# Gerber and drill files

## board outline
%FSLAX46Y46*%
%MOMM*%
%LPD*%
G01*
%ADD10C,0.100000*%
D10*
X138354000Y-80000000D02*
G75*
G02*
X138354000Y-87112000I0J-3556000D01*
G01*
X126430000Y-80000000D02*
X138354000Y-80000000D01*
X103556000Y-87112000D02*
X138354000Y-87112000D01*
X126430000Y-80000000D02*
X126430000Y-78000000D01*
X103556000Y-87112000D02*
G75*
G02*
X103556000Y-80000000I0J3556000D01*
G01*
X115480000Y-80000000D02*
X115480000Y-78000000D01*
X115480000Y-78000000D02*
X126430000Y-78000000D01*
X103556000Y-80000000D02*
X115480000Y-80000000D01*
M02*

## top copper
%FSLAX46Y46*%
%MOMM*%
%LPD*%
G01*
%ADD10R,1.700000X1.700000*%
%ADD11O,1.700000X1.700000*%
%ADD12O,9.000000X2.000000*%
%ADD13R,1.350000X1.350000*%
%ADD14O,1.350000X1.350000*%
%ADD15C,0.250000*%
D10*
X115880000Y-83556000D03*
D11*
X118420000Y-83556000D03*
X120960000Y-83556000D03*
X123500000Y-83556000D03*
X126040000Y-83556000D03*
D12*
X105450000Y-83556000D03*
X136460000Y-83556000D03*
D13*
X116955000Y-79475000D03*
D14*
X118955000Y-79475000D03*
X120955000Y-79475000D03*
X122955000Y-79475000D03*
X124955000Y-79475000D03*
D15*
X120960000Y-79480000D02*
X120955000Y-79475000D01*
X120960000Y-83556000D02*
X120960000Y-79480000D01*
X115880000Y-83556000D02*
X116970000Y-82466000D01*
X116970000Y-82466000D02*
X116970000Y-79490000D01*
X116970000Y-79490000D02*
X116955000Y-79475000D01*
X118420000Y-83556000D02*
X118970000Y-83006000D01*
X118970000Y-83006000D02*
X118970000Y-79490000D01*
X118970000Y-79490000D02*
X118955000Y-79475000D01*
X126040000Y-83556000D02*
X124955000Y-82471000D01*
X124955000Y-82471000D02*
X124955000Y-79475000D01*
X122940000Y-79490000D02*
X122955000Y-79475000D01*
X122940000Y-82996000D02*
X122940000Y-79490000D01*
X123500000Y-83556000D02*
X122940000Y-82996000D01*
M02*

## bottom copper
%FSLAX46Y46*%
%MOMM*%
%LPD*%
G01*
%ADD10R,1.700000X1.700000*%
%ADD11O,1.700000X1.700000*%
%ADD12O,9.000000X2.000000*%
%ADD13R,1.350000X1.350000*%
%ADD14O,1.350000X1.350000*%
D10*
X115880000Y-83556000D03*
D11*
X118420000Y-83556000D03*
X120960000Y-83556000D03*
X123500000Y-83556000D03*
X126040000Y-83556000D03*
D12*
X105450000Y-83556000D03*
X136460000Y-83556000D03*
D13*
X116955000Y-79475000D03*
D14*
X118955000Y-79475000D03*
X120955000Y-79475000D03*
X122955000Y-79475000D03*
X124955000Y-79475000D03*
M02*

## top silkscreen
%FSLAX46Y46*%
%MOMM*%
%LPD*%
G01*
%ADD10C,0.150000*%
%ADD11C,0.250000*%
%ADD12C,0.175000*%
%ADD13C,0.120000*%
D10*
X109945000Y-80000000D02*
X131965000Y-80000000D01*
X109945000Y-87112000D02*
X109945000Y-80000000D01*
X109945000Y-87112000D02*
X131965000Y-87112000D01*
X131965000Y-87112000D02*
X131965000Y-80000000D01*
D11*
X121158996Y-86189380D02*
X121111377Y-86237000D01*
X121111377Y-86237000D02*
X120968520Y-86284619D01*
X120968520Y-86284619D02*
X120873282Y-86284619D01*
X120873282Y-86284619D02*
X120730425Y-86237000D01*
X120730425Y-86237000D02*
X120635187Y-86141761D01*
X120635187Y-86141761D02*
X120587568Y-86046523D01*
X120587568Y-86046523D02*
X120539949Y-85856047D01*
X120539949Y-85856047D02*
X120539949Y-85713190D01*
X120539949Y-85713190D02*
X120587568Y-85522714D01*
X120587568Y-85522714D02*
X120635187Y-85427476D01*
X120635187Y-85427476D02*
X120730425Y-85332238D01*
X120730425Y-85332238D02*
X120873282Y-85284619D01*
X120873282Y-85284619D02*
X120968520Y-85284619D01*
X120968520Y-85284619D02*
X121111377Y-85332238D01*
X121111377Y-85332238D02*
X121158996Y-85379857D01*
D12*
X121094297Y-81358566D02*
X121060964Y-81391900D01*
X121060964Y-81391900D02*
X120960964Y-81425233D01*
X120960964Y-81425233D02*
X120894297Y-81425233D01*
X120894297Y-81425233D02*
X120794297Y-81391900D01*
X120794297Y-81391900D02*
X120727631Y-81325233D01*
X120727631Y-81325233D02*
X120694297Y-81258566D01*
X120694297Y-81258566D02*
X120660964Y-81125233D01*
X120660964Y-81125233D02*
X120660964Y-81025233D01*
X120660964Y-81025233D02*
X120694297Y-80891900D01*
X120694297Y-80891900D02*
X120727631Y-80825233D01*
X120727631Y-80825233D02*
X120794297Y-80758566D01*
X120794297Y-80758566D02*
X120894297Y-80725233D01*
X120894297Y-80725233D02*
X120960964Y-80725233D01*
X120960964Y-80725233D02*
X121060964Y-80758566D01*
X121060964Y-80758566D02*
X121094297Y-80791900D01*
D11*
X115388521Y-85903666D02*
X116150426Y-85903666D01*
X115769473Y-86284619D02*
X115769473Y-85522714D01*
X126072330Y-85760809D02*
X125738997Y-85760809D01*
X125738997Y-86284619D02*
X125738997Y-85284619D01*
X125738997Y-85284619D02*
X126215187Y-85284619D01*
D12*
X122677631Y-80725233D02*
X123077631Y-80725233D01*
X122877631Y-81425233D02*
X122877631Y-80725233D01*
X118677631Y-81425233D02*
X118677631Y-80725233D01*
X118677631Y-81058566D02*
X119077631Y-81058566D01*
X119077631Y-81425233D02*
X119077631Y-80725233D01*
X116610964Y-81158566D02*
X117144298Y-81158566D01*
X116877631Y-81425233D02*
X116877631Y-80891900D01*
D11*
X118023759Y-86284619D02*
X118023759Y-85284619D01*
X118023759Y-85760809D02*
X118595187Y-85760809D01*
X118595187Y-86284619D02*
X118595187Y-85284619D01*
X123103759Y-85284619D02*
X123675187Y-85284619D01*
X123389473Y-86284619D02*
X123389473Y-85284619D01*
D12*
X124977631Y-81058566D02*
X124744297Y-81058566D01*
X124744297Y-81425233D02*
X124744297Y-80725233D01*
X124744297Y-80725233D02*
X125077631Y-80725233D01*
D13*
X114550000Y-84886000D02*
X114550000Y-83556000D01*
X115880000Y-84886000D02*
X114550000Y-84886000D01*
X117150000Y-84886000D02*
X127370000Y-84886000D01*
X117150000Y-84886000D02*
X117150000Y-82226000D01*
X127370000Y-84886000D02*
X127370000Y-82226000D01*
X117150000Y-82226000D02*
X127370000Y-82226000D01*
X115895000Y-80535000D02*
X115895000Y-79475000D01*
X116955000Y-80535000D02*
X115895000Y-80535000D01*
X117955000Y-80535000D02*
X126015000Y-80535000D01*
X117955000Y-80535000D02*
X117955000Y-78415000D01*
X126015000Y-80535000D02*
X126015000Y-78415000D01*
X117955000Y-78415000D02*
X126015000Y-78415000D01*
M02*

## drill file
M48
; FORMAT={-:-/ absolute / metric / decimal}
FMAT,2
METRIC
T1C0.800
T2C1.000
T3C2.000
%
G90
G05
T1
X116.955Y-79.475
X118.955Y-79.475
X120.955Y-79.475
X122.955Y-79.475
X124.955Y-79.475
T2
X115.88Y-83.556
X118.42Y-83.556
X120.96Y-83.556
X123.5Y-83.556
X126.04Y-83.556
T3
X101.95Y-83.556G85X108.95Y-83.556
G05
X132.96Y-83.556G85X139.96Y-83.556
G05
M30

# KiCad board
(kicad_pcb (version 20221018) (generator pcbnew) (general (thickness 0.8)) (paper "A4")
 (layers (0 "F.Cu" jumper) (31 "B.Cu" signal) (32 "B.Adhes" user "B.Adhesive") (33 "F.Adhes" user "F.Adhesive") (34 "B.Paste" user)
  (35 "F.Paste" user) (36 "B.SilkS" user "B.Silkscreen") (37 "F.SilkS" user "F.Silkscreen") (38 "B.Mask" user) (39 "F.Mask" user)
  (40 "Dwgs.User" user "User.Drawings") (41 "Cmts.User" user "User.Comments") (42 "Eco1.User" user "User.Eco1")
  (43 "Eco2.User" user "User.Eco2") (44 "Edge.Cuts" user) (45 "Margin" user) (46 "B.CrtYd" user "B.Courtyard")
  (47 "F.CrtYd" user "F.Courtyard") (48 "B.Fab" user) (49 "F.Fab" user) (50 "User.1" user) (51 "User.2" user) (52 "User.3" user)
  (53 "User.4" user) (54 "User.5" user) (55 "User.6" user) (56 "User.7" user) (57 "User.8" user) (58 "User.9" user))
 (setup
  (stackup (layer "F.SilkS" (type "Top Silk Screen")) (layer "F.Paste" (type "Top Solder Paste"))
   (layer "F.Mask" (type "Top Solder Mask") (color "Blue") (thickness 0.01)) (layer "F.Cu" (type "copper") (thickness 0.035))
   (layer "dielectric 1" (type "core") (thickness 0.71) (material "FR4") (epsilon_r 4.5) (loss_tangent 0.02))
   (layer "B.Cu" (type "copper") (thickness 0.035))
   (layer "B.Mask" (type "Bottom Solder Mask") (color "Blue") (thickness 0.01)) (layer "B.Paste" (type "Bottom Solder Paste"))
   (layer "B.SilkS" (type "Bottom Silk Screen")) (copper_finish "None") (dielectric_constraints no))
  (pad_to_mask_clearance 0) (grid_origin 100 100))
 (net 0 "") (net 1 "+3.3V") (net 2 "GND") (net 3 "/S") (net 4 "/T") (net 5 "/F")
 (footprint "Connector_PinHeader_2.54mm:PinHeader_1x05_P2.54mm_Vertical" (layer "F.Cu") (at 115.88 83.556 90)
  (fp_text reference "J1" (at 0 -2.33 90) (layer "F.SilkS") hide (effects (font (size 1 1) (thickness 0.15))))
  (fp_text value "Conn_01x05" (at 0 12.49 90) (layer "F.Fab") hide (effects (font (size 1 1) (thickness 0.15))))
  (fp_line (start -1.33 -1.33) (end 0 -1.33) (stroke (width 0.12) (type solid)) (layer "F.SilkS"))
  (fp_line (start -1.33 0) (end -1.33 -1.33) (stroke (width 0.12) (type solid)) (layer "F.SilkS"))
  (fp_line (start -1.33 1.27) (end -1.33 11.49) (stroke (width 0.12) (type solid)) (layer "F.SilkS"))
  (fp_line (start -1.33 1.27) (end 1.33 1.27) (stroke (width 0.12) (type solid)) (layer "F.SilkS"))
  (fp_line (start -1.33 11.49) (end 1.33 11.49) (stroke (width 0.12) (type solid)) (layer "F.SilkS"))
  (fp_line (start 1.33 1.27) (end 1.33 11.49) (stroke (width 0.12) (type solid)) (layer "F.SilkS"))
  (pad "1" thru_hole rect (at 0 0 90) (size 1.7 1.7) (drill 1) (layers "*.Cu" "*.Mask") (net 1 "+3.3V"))
  (pad "2" thru_hole oval (at 0 2.54 90) (size 1.7 1.7) (drill 1) (layers "*.Cu" "*.Mask") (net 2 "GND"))
  (pad "3" thru_hole oval (at 0 5.08 90) (size 1.7 1.7) (drill 1) (layers "*.Cu" "*.Mask") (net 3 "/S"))
  (pad "4" thru_hole oval (at 0 7.62 90) (size 1.7 1.7) (drill 1) (layers "*.Cu" "*.Mask") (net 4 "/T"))
  (pad "5" thru_hole oval (at 0 10.16 90) (size 1.7 1.7) (drill 1) (layers "*.Cu" "*.Mask") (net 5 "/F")))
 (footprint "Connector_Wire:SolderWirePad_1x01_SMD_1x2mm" (layer "F.Cu") (at 105.45 83.556)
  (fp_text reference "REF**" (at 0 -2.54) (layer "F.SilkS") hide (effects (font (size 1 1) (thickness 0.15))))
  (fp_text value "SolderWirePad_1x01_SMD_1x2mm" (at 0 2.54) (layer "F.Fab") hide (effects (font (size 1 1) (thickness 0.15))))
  (pad "1" thru_hole oval (at 0 0) (size 9 2) (drill oval 9 2) (layers "*.Cu" "*.Mask")))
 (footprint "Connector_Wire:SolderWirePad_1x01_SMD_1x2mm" (layer "F.Cu") (at 136.46 83.556)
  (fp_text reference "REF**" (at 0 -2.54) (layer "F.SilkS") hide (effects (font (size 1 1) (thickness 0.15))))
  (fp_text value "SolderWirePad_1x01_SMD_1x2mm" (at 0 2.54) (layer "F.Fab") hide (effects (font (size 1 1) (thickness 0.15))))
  (pad "1" thru_hole oval (at 0 0) (size 9 2) (drill oval 9 2) (layers "*.Cu" "*.Mask")))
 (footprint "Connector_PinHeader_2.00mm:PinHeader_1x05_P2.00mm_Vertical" (layer "F.Cu") (at 116.955 79.475 90)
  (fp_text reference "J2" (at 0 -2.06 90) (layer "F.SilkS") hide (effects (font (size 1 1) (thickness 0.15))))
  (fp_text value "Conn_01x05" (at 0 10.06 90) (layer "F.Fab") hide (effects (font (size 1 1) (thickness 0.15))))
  (fp_line (start -1.06 -1.06) (end 0 -1.06) (stroke (width 0.12) (type solid)) (layer "F.SilkS"))
  (fp_line (start -1.06 0) (end -1.06 -1.06) (stroke (width 0.12) (type solid)) (layer "F.SilkS"))
  (fp_line (start -1.06 1) (end -1.06 9.06) (stroke (width 0.12) (type solid)) (layer "F.SilkS"))
  (fp_line (start -1.06 1) (end 1.06 1) (stroke (width 0.12) (type solid)) (layer "F.SilkS"))
  (fp_line (start -1.06 9.06) (end 1.06 9.06) (stroke (width 0.12) (type solid)) (layer "F.SilkS"))
  (fp_line (start 1.06 1) (end 1.06 9.06) (stroke (width 0.12) (type solid)) (layer "F.SilkS"))
  (pad "1" thru_hole rect (at 0 0 90) (size 1.35 1.35) (drill 0.8) (layers "*.Cu" "*.Mask") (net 1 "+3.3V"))
  (pad "2" thru_hole oval (at 0 2 90) (size 1.35 1.35) (drill 0.8) (layers "*.Cu" "*.Mask") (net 2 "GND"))
  (pad "3" thru_hole oval (at 0 4 90) (size 1.35 1.35) (drill 0.8) (layers "*.Cu" "*.Mask") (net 3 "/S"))
  (pad "4" thru_hole oval (at 0 6 90) (size 1.35 1.35) (drill 0.8) (layers "*.Cu" "*.Mask") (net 4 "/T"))
  (pad "5" thru_hole oval (at 0 8 90) (size 1.35 1.35) (drill 0.8) (layers "*.Cu" "*.Mask") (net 5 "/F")))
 (gr_line (start 109.945 80) (end 131.965 80) (stroke (width 0.15) (type default)) (layer "F.SilkS"))
 (gr_line (start 109.945 87.112) (end 109.945 80) (stroke (width 0.15) (type default)) (layer "F.SilkS"))
 (gr_line (start 109.945 87.112) (end 131.965 87.112) (stroke (width 0.15) (type default)) (layer "F.SilkS"))
 (gr_line (start 131.965 87.112) (end 131.965 80) (stroke (width 0.15) (type default)) (layer "F.SilkS"))
 (gr_arc (start 138.354 80) (mid 141.91 83.556) (end 138.354 87.112) (stroke (width 0.1) (type default)) (layer "Edge.Cuts"))
 (gr_line (start 126.43 80) (end 138.354 80) (stroke (width 0.1) (type default)) (layer "Edge.Cuts"))
 (gr_line (start 103.556 87.112) (end 138.354 87.112) (stroke (width 0.1) (type default)) (layer "Edge.Cuts"))
 (gr_line (start 126.43 80) (end 126.43 78) (stroke (width 0.1) (type default)) (layer "Edge.Cuts"))
 (gr_arc (start 103.556 87.112) (mid 100 83.556) (end 103.556 80) (stroke (width 0.1) (type default)) (layer "Edge.Cuts"))
 (gr_line (start 115.48 80) (end 115.48 78) (stroke (width 0.1) (type default)) (layer "Edge.Cuts"))
 (gr_line (start 115.48 78) (end 126.43 78) (stroke (width 0.1) (type default)) (layer "Edge.Cuts"))
 (gr_line (start 103.556 80) (end 115.48 80) (stroke (width 0.1) (type default)) (layer "Edge.Cuts"))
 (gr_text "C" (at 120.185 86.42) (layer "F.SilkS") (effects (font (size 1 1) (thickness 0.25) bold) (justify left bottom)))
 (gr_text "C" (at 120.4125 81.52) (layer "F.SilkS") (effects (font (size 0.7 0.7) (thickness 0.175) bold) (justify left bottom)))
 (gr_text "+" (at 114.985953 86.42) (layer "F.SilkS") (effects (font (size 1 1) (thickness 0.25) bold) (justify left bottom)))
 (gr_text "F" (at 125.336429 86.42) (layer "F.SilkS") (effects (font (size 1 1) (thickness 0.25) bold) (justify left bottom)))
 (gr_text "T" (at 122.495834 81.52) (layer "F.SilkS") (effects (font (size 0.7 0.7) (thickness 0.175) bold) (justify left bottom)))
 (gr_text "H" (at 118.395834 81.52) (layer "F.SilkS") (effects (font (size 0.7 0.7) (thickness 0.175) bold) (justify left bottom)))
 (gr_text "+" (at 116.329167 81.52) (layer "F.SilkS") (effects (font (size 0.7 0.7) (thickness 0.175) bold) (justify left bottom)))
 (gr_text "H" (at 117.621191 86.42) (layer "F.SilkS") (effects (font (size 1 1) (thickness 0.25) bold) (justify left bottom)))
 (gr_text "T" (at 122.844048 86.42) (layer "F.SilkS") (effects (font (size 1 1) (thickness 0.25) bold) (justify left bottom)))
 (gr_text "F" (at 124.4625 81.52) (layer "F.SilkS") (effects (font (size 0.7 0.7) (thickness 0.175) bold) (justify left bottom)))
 (segment (start 120.96 79.48) (end 120.955 79.475) (width 0.25) (layer "F.Cu") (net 3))
 (segment (start 120.96 83.556) (end 120.96 79.48) (width 0.25) (layer "F.Cu") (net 3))
 (segment (start 115.88 83.556) (end 116.97 82.466) (width 0.25) (layer "F.Cu") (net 1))
 (segment (start 116.97 82.466) (end 116.97 79.49) (width 0.25) (layer "F.Cu") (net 1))
 (segment (start 116.97 79.49) (end 116.955 79.475) (width 0.25) (layer "F.Cu") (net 1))
 (segment (start 118.42 83.556) (end 118.97 83.006) (width 0.25) (layer "F.Cu") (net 2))
 (segment (start 118.97 83.006) (end 118.97 79.49) (width 0.25) (layer "F.Cu") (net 2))
 (segment (start 118.97 79.49) (end 118.955 79.475) (width 0.25) (layer "F.Cu") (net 2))
 (segment (start 126.04 83.556) (end 124.955 82.471) (width 0.25) (layer "F.Cu") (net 5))
 (segment (start 124.955 82.471) (end 124.955 79.475) (width 0.25) (layer "F.Cu") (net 5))
 (segment (start 122.94 79.49) (end 122.955 79.475) (width 0.25) (layer "F.Cu") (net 4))
 (segment (start 122.94 82.996) (end 122.94 79.49) (width 0.25) (layer "F.Cu") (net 4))
 (segment (start 123.5 83.556) (end 122.94 82.996) (width 0.25) (layer "F.Cu") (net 4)))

